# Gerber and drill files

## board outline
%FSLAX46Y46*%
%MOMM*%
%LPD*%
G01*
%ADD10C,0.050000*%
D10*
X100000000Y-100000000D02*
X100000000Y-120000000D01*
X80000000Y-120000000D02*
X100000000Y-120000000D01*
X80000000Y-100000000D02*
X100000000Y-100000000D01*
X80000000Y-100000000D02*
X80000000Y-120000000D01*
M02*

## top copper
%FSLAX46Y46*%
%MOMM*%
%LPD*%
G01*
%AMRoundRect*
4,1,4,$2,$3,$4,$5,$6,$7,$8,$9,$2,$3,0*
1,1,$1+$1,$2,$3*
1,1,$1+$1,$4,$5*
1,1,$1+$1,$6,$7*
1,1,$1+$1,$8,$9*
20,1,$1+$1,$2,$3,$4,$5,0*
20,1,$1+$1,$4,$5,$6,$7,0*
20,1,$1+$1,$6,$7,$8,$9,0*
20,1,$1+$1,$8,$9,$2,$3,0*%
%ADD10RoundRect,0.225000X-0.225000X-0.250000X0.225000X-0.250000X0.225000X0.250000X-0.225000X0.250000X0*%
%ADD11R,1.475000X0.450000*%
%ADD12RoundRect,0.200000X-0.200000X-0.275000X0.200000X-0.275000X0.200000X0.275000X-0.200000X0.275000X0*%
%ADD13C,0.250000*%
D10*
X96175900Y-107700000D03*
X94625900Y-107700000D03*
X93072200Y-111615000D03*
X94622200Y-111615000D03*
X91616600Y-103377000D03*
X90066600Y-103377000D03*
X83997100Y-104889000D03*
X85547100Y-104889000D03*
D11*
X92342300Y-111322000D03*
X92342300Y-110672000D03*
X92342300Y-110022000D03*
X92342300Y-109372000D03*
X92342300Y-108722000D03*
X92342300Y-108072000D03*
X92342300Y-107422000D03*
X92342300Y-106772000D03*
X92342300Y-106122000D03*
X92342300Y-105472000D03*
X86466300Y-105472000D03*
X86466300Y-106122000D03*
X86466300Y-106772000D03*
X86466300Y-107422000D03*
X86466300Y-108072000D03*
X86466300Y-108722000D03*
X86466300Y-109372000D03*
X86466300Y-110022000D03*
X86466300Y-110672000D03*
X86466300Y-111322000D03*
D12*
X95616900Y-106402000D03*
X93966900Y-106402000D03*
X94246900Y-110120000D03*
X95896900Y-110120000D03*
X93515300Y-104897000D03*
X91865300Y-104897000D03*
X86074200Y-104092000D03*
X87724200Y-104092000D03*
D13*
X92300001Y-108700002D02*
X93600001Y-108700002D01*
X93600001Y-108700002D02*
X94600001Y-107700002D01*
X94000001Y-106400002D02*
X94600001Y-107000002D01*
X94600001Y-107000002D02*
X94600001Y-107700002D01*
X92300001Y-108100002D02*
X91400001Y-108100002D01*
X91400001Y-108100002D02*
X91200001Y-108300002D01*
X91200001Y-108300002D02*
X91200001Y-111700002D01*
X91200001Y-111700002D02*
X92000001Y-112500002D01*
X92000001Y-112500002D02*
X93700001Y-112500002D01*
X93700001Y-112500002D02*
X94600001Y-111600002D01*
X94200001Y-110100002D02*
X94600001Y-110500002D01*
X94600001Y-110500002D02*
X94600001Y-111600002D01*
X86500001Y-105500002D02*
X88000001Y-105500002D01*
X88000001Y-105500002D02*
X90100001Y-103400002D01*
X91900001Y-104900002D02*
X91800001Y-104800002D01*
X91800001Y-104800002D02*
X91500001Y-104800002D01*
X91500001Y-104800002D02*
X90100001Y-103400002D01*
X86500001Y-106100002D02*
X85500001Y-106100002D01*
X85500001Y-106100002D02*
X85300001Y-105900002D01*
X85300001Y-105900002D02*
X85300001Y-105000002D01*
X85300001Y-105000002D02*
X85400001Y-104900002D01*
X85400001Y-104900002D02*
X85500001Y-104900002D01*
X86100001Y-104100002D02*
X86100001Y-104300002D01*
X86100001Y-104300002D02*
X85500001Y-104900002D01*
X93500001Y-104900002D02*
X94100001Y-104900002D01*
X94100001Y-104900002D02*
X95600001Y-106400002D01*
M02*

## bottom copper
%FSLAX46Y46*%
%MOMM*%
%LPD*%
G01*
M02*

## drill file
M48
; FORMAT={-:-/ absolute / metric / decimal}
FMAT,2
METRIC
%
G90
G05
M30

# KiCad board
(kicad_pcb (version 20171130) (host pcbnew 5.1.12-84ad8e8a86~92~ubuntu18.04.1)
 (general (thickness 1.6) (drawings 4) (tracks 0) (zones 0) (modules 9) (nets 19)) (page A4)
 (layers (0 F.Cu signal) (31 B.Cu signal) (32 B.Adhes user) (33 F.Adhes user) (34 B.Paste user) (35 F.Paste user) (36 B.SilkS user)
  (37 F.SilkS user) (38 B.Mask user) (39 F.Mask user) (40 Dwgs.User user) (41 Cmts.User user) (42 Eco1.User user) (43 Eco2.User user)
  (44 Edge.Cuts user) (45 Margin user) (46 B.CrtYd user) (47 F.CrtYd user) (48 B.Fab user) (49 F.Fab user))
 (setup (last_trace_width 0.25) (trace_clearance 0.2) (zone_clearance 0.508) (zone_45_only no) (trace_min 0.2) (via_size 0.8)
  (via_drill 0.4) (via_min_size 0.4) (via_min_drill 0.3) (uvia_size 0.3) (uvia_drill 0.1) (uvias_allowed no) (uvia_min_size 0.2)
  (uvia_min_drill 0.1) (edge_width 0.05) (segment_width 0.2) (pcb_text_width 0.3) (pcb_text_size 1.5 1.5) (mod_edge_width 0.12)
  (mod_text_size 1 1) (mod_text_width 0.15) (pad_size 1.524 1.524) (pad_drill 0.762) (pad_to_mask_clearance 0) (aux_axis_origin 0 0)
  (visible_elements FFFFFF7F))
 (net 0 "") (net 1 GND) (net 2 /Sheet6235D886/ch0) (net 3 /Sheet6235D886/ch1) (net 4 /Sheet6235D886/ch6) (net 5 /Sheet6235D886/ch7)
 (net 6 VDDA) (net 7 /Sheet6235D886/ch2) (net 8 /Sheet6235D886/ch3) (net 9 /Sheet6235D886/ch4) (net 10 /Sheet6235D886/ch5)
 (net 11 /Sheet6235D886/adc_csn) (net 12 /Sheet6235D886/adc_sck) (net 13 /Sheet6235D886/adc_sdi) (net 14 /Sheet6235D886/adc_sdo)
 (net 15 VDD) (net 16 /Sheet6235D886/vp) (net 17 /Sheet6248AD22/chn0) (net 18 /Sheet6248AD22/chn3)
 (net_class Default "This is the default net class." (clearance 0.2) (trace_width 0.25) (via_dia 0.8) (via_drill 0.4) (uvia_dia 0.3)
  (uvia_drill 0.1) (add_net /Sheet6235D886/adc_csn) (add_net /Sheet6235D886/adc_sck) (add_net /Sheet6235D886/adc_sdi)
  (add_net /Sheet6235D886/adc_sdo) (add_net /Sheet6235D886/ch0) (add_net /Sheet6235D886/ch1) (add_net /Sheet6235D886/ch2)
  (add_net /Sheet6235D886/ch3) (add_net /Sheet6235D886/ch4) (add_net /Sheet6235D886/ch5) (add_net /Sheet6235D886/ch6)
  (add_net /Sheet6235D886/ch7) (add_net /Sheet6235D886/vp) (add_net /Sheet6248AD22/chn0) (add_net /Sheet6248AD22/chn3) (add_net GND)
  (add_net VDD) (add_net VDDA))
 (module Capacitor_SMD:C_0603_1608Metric (layer F.Cu) (at 95.400900 107.700000)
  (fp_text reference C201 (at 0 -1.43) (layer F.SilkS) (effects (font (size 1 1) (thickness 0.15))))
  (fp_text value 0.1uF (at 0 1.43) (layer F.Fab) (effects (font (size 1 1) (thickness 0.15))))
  (pad 2 smd roundrect (at 0.775 0) (size 0.9 0.95) (layers F.Cu F.Mask F.Paste) (roundrect_rratio 0.25) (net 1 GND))
  (pad 1 smd roundrect (at -0.775 0) (size 0.9 0.95) (layers F.Cu F.Mask F.Paste) (roundrect_rratio 0.25) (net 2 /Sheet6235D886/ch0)))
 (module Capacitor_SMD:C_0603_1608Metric (layer F.Cu) (at 93.847200 111.615000)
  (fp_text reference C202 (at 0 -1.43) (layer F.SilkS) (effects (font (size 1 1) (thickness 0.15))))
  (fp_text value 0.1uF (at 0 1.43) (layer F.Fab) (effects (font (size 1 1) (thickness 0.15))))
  (pad 1 smd roundrect (at -0.775 0) (size 0.9 0.95) (layers F.Cu F.Mask F.Paste) (roundrect_rratio 0.25) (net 1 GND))
  (pad 2 smd roundrect (at 0.775 0) (size 0.9 0.95) (layers F.Cu F.Mask F.Paste) (roundrect_rratio 0.25) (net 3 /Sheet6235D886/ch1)))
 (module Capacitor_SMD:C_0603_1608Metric (layer F.Cu) (at 90.841600 103.377000)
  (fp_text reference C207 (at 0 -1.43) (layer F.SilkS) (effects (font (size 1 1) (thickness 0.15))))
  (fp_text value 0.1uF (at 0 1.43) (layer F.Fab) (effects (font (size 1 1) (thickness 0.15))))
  (pad 2 smd roundrect (at 0.775 0) (size 0.9 0.95) (layers F.Cu F.Mask F.Paste) (roundrect_rratio 0.25) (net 1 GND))
  (pad 1 smd roundrect (at -0.775 0) (size 0.9 0.95) (layers F.Cu F.Mask F.Paste) (roundrect_rratio 0.25) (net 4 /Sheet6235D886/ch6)))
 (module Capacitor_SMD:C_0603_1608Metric (layer F.Cu) (at 84.772100 104.889000)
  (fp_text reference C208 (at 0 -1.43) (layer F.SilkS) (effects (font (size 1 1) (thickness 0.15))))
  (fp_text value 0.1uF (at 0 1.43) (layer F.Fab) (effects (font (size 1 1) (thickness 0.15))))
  (pad 1 smd roundrect (at -0.775 0) (size 0.9 0.95) (layers F.Cu F.Mask F.Paste) (roundrect_rratio 0.25) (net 1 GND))
  (pad 2 smd roundrect (at 0.775 0) (size 0.9 0.95) (layers F.Cu F.Mask F.Paste) (roundrect_rratio 0.25) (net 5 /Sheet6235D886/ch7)))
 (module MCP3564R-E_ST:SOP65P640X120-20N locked (layer F.Cu) (at 89.404300 108.397000 180.000000)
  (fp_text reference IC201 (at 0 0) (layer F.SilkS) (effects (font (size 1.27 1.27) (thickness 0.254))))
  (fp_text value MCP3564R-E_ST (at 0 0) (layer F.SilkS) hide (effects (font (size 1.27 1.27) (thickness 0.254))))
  (pad 1 smd rect (at -2.938 -2.925 270.000000) (size 0.45 1.475) (layers F.Cu F.Mask F.Paste) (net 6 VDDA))
  (pad 2 smd rect (at -2.938 -2.275 270.000000) (size 0.45 1.475) (layers F.Cu F.Mask F.Paste) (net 1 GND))
  (pad 3 smd rect (at -2.938 -1.625 270.000000) (size 0.45 1.475) (layers F.Cu F.Mask F.Paste) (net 1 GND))
  (pad 4 smd rect (at -2.938 -0.975 270.000000) (size 0.45 1.475) (layers F.Cu F.Mask F.Paste))
  (pad 5 smd rect (at -2.938 -0.325 270.000000) (size 0.45 1.475) (layers F.Cu F.Mask F.Paste) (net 2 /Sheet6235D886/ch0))
  (pad 6 smd rect (at -2.938 0.325 270.000000) (size 0.45 1.475) (layers F.Cu F.Mask F.Paste) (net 3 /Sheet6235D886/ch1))
  (pad 7 smd rect (at -2.938 0.975 270.000000) (size 0.45 1.475) (layers F.Cu F.Mask F.Paste) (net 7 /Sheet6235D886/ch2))
  (pad 8 smd rect (at -2.938 1.625 270.000000) (size 0.45 1.475) (layers F.Cu F.Mask F.Paste) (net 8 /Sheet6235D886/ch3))
  (pad 9 smd rect (at -2.938 2.275 270.000000) (size 0.45 1.475) (layers F.Cu F.Mask F.Paste) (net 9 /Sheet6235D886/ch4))
  (pad 10 smd rect (at -2.938 2.925 270.000000) (size 0.45 1.475) (layers F.Cu F.Mask F.Paste) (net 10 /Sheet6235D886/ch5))
  (pad 11 smd rect (at 2.938 2.925 270.000000) (size 0.45 1.475) (layers F.Cu F.Mask F.Paste) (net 4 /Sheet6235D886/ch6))
  (pad 12 smd rect (at 2.938 2.275 270.000000) (size 0.45 1.475) (layers F.Cu F.Mask F.Paste) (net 5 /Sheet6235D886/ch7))
  (pad 13 smd rect (at 2.938 1.625 270.000000) (size 0.45 1.475) (layers F.Cu F.Mask F.Paste) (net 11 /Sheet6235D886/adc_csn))
  (pad 14 smd rect (at 2.938 0.975 270.000000) (size 0.45 1.475) (layers F.Cu F.Mask F.Paste) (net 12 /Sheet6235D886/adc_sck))
  (pad 15 smd rect (at 2.938 0.325 270.000000) (size 0.45 1.475) (layers F.Cu F.Mask F.Paste) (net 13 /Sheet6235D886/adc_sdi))
  (pad 16 smd rect (at 2.938 -0.325 270.000000) (size 0.45 1.475) (layers F.Cu F.Mask F.Paste) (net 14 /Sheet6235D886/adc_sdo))
  (pad 17 smd rect (at 2.938 -0.975 270.000000) (size 0.45 1.475) (layers F.Cu F.Mask F.Paste))
  (pad 18 smd rect (at 2.938 -1.625 270.000000) (size 0.45 1.475) (layers F.Cu F.Mask F.Paste))
  (pad 19 smd rect (at 2.938 -2.275 270.000000) (size 0.45 1.475) (layers F.Cu F.Mask F.Paste) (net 1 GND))
  (pad 20 smd rect (at 2.938 -2.925 270.000000) (size 0.45 1.475) (layers F.Cu F.Mask F.Paste) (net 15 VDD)))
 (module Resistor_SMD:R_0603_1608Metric (layer F.Cu) (at 94.791900 106.402000)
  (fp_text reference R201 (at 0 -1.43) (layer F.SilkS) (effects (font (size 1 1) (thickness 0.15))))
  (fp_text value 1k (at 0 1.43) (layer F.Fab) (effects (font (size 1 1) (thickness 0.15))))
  (pad 2 smd roundrect (at 0.825 0) (size 0.8 0.95) (layers F.Cu F.Mask F.Paste) (roundrect_rratio 0.25) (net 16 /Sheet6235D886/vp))
  (pad 1 smd roundrect (at -0.825 0) (size 0.8 0.95) (layers F.Cu F.Mask F.Paste) (roundrect_rratio 0.25) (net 2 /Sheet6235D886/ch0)))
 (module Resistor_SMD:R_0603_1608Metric (layer F.Cu) (at 95.071900 110.120000)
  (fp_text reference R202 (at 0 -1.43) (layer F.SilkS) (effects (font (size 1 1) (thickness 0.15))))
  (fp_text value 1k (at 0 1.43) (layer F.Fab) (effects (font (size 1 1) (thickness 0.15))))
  (pad 1 smd roundrect (at -0.825 0) (size 0.8 0.95) (layers F.Cu F.Mask F.Paste) (roundrect_rratio 0.25) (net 3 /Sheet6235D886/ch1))
  (pad 2 smd roundrect (at 0.825 0) (size 0.8 0.95) (layers F.Cu F.Mask F.Paste) (roundrect_rratio 0.25) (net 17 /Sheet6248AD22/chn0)))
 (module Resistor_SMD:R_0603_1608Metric (layer F.Cu) (at 92.690300 104.897000)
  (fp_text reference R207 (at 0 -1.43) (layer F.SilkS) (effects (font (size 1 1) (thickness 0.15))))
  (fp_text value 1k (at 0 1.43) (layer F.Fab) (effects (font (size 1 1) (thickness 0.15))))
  (pad 2 smd roundrect (at 0.825 0) (size 0.8 0.95) (layers F.Cu F.Mask F.Paste) (roundrect_rratio 0.25) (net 16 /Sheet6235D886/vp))
  (pad 1 smd roundrect (at -0.825 0) (size 0.8 0.95) (layers F.Cu F.Mask F.Paste) (roundrect_rratio 0.25) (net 4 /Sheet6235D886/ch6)))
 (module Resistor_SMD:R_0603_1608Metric (layer F.Cu) (at 86.899200 104.092000)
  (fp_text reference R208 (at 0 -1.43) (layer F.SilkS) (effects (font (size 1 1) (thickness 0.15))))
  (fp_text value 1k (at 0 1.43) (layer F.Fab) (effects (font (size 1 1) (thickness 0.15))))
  (pad 1 smd roundrect (at -0.825 0) (size 0.8 0.95) (layers F.Cu F.Mask F.Paste) (roundrect_rratio 0.25) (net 5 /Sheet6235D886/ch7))
  (pad 2 smd roundrect (at 0.825 0) (size 0.8 0.95) (layers F.Cu F.Mask F.Paste) (roundrect_rratio 0.25) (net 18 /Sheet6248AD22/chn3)))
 (gr_line (start 100 100) (end 100 120) (layer Edge.Cuts) (width 0.05))
 (gr_line (start 80 120) (end 100 120) (layer Edge.Cuts) (width 0.05))
 (gr_line (start 80 100) (end 100 100) (layer Edge.Cuts) (width 0.05))
 (gr_line (start 80 100) (end 80 120) (layer Edge.Cuts) (width 0.05))
 (segment (start 92.300001 108.700002) (end 93.600001 108.700002) (width 0.250000) (layer F.Cu) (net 2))
 (segment (start 93.600001 108.700002) (end 94.600001 107.700002) (width 0.250000) (layer F.Cu) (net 2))
 (segment (start 94.000001 106.400002) (end 94.600001 107.000002) (width 0.250000) (layer F.Cu) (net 2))
 (segment (start 94.600001 107.000002) (end 94.600001 107.700002) (width 0.250000) (layer F.Cu) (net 2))
 (segment (start 92.300001 108.100002) (end 91.400001 108.100002) (width 0.250000) (layer F.Cu) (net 3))
 (segment (start 91.400001 108.100002) (end 91.200001 108.300002) (width 0.250000) (layer F.Cu) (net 3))
 (segment (start 91.200001 108.300002) (end 91.200001 111.700002) (width 0.250000) (layer F.Cu) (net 3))
 (segment (start 91.200001 111.700002) (end 92.000001 112.500002) (width 0.250000) (layer F.Cu) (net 3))
 (segment (start 92.000001 112.500002) (end 93.700001 112.500002) (width 0.250000) (layer F.Cu) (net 3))
 (segment (start 93.700001 112.500002) (end 94.600001 111.600002) (width 0.250000) (layer F.Cu) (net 3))
 (segment (start 94.200001 110.100002) (end 94.600001 110.500002) (width 0.250000) (layer F.Cu) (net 3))
 (segment (start 94.600001 110.500002) (end 94.600001 111.600002) (width 0.250000) (layer F.Cu) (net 3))
 (segment (start 86.500001 105.500002) (end 88.000001 105.500002) (width 0.250000) (layer F.Cu) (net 4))
 (segment (start 88.000001 105.500002) (end 90.100001 103.400002) (width 0.250000) (layer F.Cu) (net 4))
 (segment (start 91.900001 104.900002) (end 91.800001 104.800002) (width 0.250000) (layer F.Cu) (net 4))
 (segment (start 91.800001 104.800002) (end 91.500001 104.800002) (width 0.250000) (layer F.Cu) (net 4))
 (segment (start 91.500001 104.800002) (end 90.100001 103.400002) (width 0.250000) (layer F.Cu) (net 4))
 (segment (start 86.500001 106.100002) (end 85.500001 106.100002) (width 0.250000) (layer F.Cu) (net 5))
 (segment (start 85.500001 106.100002) (end 85.300001 105.900002) (width 0.250000) (layer F.Cu) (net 5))
 (segment (start 85.300001 105.900002) (end 85.300001 105.000002) (width 0.250000) (layer F.Cu) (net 5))
 (segment (start 85.300001 105.000002) (end 85.400001 104.900002) (width 0.250000) (layer F.Cu) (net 5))
 (segment (start 85.400001 104.900002) (end 85.500001 104.900002) (width 0.250000) (layer F.Cu) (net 5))
 (segment (start 86.100001 104.100002) (end 86.100001 104.300002) (width 0.250000) (layer F.Cu) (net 5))
 (segment (start 86.100001 104.300002) (end 85.500001 104.900002) (width 0.250000) (layer F.Cu) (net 5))
 (segment (start 93.500001 104.900002) (end 94.100001 104.900002) (width 0.250000) (layer F.Cu) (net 16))
 (segment (start 94.100001 104.900002) (end 95.600001 106.400002) (width 0.250000) (layer F.Cu) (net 16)))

